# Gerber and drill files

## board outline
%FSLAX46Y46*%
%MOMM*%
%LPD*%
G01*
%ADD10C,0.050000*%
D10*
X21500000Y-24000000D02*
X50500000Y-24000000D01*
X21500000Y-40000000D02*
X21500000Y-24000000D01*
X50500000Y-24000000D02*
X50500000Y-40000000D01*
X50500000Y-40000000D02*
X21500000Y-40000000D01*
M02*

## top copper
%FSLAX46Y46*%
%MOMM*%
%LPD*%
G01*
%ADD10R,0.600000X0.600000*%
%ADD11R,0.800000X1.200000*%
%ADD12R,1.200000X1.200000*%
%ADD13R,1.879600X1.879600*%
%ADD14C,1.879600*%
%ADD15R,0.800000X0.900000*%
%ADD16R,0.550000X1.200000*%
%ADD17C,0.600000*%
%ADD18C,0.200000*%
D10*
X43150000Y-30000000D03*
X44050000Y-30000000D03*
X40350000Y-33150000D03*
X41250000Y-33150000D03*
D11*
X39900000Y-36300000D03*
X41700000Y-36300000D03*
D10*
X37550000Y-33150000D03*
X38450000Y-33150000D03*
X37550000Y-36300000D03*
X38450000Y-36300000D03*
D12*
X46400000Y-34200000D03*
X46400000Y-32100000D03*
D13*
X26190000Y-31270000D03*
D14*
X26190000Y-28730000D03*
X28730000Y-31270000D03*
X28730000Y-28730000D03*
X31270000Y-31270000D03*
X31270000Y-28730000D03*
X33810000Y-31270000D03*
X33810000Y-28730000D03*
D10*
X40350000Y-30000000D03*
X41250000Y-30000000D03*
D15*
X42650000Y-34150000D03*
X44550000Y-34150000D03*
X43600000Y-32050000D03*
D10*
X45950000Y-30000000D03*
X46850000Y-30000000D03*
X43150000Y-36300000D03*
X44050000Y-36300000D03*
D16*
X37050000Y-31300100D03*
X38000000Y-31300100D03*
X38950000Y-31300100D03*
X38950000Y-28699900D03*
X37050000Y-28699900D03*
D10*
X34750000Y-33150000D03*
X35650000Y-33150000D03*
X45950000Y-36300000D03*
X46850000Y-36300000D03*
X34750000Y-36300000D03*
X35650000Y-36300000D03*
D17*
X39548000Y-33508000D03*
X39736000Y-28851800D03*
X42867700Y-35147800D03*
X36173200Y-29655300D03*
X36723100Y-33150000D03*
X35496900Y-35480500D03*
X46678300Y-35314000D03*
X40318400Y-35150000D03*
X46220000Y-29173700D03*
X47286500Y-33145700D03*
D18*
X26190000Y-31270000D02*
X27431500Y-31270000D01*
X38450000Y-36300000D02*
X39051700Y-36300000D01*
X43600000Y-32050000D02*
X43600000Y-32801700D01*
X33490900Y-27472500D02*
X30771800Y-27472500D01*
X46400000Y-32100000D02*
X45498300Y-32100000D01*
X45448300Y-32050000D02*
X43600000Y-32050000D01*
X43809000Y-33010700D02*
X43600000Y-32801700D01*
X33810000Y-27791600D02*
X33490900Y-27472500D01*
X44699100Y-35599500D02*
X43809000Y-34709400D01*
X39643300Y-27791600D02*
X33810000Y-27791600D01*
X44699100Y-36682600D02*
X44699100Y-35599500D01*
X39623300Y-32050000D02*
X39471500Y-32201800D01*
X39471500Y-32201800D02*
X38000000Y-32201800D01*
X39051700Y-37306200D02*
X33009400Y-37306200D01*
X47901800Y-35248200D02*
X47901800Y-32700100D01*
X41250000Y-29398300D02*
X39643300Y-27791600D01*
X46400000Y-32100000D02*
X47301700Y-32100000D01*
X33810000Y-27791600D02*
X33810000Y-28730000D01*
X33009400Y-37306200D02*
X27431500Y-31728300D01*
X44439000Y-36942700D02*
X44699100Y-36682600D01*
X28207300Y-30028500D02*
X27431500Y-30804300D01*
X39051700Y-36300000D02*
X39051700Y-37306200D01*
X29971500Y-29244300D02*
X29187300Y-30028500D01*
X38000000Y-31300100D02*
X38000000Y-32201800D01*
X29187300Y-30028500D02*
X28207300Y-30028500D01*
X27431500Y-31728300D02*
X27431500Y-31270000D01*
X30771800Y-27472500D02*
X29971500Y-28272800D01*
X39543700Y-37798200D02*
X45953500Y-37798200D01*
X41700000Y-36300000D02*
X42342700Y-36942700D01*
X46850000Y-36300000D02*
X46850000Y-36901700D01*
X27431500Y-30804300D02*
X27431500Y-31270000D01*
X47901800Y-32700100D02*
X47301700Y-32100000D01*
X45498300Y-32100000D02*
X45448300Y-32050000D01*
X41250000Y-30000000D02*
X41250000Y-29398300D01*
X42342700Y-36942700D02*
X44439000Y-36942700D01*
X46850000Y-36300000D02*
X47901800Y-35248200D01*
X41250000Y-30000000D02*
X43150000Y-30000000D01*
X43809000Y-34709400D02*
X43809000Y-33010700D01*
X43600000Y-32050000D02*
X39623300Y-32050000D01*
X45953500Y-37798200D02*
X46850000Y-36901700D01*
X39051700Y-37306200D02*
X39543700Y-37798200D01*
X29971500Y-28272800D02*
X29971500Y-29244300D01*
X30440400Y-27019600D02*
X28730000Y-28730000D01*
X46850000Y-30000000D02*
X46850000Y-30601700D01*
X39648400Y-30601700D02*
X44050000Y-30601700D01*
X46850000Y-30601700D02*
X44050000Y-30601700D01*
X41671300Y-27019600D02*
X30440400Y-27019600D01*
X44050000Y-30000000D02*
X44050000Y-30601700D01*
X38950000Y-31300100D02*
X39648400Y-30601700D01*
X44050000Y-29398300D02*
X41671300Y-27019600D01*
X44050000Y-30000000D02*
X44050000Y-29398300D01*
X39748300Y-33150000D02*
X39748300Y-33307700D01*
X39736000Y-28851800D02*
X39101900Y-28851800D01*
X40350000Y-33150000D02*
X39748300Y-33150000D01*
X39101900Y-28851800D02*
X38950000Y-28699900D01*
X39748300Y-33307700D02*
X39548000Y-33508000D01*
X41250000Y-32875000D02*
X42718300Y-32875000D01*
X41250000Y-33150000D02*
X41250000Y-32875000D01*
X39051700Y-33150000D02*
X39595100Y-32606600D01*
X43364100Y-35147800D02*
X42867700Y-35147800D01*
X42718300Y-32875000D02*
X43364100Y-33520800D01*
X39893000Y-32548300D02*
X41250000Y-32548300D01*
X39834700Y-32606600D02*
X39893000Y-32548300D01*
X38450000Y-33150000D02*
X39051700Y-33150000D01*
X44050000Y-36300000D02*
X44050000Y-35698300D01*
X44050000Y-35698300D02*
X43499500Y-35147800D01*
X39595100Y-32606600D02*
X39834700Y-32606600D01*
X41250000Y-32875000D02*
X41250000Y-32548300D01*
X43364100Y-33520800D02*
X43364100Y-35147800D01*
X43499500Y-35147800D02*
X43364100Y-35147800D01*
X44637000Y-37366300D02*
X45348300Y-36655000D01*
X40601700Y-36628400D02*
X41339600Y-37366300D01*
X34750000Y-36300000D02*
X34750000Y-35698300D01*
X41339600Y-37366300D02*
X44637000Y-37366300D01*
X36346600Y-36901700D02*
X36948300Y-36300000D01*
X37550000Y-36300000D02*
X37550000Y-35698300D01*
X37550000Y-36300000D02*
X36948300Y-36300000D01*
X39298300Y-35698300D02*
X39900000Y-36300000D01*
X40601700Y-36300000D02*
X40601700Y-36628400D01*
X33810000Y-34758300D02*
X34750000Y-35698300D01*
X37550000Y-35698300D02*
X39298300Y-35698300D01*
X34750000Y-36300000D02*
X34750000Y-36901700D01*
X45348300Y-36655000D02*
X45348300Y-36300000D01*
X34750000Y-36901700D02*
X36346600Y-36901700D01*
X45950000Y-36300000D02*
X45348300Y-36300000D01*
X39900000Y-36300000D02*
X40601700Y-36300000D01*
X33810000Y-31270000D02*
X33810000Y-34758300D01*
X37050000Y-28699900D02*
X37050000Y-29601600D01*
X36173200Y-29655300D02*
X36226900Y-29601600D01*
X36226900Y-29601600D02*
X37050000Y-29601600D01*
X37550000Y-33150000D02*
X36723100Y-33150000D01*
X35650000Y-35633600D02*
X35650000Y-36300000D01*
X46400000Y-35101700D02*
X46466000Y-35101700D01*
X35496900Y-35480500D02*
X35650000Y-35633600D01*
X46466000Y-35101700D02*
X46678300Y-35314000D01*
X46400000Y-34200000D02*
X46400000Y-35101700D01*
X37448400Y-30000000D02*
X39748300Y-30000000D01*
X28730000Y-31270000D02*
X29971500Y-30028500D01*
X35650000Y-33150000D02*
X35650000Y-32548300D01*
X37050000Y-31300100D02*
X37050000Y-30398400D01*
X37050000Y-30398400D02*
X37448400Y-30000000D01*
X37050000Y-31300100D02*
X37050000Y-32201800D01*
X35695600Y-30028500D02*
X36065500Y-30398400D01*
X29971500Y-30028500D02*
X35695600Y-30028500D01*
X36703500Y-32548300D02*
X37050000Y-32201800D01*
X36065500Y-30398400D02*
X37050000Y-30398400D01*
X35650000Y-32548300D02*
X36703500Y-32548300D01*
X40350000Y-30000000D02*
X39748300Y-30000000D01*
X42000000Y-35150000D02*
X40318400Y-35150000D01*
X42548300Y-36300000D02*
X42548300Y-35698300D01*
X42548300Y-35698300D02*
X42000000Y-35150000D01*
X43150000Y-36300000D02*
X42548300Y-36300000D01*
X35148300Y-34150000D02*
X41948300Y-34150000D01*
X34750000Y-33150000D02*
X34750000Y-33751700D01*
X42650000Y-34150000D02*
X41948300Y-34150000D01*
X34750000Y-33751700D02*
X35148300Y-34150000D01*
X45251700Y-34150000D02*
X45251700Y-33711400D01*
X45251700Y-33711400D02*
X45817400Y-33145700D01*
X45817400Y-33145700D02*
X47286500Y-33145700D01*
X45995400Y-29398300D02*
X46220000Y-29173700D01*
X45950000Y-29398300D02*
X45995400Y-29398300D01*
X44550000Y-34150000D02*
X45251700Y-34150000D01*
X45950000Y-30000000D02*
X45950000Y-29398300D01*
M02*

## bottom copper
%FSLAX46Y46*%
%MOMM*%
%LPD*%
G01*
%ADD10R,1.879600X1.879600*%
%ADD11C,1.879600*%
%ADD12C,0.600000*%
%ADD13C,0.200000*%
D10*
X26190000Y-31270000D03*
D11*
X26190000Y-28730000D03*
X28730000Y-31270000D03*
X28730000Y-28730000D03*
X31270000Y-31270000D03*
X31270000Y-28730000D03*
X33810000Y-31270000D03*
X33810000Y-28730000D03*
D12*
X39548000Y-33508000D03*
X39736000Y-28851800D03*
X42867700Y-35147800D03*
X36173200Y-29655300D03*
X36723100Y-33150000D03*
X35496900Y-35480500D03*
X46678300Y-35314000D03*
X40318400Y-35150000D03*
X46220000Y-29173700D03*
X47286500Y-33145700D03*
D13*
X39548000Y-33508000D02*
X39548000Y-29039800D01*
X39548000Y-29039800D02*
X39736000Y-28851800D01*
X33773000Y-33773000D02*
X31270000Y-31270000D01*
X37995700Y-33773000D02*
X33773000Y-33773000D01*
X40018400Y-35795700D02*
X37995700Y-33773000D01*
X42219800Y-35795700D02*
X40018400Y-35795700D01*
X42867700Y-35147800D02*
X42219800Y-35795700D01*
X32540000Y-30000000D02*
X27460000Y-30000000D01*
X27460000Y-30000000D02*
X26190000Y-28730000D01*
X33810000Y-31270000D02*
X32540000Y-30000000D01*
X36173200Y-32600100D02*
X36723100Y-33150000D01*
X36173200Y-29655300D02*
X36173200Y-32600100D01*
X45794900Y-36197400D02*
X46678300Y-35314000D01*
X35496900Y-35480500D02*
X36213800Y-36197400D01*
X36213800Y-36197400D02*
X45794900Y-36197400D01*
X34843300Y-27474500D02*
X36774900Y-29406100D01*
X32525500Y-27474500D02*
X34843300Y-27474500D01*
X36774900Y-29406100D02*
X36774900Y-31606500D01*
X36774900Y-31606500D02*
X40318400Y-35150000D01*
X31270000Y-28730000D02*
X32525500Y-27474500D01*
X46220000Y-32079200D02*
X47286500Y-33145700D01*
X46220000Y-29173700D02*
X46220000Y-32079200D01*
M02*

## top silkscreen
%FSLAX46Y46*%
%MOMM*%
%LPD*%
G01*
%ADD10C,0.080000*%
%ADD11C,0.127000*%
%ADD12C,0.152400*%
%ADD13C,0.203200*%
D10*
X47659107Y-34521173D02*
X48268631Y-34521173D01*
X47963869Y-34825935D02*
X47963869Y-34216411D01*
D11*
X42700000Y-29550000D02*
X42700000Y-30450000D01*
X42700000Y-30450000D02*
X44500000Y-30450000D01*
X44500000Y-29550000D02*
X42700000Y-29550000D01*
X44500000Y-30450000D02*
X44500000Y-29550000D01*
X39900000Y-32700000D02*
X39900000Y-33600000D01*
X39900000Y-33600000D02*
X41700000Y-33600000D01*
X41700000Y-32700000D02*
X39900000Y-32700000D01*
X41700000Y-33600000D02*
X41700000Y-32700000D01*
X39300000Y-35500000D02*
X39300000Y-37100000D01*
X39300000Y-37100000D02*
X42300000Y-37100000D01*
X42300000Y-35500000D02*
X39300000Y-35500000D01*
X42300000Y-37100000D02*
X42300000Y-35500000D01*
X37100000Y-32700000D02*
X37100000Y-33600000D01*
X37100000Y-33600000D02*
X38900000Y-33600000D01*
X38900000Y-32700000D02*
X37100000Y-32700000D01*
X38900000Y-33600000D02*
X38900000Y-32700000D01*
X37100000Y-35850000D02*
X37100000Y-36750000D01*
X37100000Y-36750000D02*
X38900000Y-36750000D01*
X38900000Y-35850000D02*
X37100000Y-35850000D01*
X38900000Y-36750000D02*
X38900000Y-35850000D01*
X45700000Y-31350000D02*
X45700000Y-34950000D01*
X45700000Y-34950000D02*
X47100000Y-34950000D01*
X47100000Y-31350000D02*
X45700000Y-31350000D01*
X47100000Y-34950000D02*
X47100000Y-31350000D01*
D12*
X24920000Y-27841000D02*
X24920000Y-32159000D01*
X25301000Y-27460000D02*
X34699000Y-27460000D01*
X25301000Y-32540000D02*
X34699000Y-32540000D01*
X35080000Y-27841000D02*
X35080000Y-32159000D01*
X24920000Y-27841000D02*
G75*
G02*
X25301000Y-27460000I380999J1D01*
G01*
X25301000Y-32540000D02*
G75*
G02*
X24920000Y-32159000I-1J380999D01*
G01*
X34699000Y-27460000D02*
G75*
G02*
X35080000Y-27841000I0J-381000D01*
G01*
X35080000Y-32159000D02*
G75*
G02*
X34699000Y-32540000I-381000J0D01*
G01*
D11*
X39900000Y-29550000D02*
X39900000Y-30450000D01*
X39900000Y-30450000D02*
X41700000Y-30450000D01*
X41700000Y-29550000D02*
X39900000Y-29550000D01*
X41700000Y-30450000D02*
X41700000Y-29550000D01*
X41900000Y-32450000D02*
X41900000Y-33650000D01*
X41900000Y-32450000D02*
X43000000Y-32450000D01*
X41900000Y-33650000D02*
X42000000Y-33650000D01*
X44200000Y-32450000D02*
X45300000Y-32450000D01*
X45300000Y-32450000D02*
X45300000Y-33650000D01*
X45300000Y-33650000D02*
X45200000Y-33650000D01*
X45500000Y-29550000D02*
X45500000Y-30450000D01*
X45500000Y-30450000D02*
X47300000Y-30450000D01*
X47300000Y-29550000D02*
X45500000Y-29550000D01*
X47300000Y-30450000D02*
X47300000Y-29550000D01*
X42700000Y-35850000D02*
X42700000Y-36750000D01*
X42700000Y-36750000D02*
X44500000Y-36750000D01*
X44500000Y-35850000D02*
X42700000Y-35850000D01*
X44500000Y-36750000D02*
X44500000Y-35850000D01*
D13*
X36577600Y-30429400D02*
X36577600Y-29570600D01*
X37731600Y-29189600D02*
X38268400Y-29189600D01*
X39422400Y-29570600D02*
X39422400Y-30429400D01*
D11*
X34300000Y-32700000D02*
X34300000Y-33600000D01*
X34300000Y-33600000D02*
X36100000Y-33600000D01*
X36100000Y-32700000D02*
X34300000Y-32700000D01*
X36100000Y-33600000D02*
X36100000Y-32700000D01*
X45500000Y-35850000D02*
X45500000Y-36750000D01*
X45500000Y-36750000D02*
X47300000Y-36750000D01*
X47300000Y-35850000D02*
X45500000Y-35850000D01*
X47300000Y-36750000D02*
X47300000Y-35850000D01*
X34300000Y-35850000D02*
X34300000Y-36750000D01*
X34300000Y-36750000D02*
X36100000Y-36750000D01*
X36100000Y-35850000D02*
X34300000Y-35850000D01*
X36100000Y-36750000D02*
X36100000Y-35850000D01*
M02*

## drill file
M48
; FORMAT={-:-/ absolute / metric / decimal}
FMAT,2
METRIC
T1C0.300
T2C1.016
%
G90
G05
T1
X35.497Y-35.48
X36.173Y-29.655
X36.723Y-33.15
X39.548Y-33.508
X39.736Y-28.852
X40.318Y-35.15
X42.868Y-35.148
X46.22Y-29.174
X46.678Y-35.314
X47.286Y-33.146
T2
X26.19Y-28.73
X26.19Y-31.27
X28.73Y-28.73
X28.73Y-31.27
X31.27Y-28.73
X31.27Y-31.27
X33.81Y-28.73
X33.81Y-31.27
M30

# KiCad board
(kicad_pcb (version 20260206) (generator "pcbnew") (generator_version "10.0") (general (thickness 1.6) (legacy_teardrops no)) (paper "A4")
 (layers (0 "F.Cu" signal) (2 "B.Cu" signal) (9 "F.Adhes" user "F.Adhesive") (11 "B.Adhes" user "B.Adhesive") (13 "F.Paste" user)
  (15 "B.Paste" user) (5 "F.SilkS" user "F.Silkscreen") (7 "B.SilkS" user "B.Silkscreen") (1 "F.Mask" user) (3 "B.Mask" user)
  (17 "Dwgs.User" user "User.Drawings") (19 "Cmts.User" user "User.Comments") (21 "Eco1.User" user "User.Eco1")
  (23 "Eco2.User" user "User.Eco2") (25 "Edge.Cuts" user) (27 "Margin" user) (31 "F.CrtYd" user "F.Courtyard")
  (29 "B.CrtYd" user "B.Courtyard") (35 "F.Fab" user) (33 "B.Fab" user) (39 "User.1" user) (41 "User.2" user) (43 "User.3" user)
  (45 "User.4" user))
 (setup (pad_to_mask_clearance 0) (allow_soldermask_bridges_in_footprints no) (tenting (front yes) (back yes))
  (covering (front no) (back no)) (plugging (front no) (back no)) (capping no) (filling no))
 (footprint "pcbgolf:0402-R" (layer "F.Cu") (at 43.6 30)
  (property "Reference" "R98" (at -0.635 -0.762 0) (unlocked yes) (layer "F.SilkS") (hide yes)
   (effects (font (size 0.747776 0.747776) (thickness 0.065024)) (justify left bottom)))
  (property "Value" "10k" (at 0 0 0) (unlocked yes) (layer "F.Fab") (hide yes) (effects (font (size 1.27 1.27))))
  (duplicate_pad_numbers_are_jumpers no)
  (fp_line (start -0.9 -0.45) (end -0.9 0.45) (stroke (width 0.127) (type solid)) (layer "F.SilkS"))
  (fp_line (start -0.9 0.45) (end 0.9 0.45) (stroke (width 0.127) (type solid)) (layer "F.SilkS"))
  (fp_line (start 0.9 -0.45) (end -0.9 -0.45) (stroke (width 0.127) (type solid)) (layer "F.SilkS"))
  (fp_line (start 0.9 0.45) (end 0.9 -0.45) (stroke (width 0.127) (type solid)) (layer "F.SilkS"))
  (pad "1" smd rect (at -0.45 0) (size 0.6 0.6) (layers "F.Cu" "F.Mask" "F.Paste") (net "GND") (solder_mask_margin 0.0508)
   (solder_paste_margin 0) (thermal_bridge_angle 0))
  (pad "2" smd rect (at 0.45 0) (size 0.6 0.6) (layers "F.Cu" "F.Mask" "F.Paste") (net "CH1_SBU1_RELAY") (solder_mask_margin 0.0508)
   (solder_paste_margin 0) (thermal_bridge_angle 0)))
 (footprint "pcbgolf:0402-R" (layer "F.Cu") (at 40.8 33.15)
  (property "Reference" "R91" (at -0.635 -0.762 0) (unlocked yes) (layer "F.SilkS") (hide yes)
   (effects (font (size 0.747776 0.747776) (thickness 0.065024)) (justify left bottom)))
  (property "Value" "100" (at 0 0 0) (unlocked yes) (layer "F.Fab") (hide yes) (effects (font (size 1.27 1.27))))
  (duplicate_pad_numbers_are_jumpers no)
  (fp_line (start -0.9 -0.45) (end -0.9 0.45) (stroke (width 0.127) (type solid)) (layer "F.SilkS"))
  (fp_line (start -0.9 0.45) (end 0.9 0.45) (stroke (width 0.127) (type solid)) (layer "F.SilkS"))
  (fp_line (start 0.9 -0.45) (end -0.9 -0.45) (stroke (width 0.127) (type solid)) (layer "F.SilkS"))
  (fp_line (start 0.9 0.45) (end 0.9 -0.45) (stroke (width 0.127) (type solid)) (layer "F.SilkS"))
  (pad "1" smd rect (at -0.45 0) (size 0.6 0.6) (layers "F.Cu" "F.Mask" "F.Paste") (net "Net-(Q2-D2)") (solder_mask_margin 0.0508)
   (solder_paste_margin 0) (thermal_bridge_angle 0))
  (pad "2" smd rect (at 0.45 0) (size 0.6 0.6) (layers "F.Cu" "F.Mask" "F.Paste") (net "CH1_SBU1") (solder_mask_margin 0.0508)
   (solder_paste_margin 0) (thermal_bridge_angle 0)))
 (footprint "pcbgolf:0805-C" (layer "F.Cu") (at 40.8 36.3)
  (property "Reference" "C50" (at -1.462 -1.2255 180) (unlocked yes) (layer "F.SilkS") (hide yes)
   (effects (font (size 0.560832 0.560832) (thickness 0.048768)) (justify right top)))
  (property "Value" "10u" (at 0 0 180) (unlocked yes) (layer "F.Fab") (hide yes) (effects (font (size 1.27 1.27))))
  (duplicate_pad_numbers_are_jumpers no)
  (fp_line (start -1.5 -0.8) (end -1.5 0.8) (stroke (width 0.127) (type solid)) (layer "F.SilkS"))
  (fp_line (start -1.5 0.8) (end 1.5 0.8) (stroke (width 0.127) (type solid)) (layer "F.SilkS"))
  (fp_line (start 1.5 -0.8) (end -1.5 -0.8) (stroke (width 0.127) (type solid)) (layer "F.SilkS"))
  (fp_line (start 1.5 0.8) (end 1.5 -0.8) (stroke (width 0.127) (type solid)) (layer "F.SilkS"))
  (pad "1" smd rect (at -0.9 0) (size 0.8 1.2) (layers "F.Cu" "F.Mask" "F.Paste") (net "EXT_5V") (solder_mask_margin 0.0508)
   (solder_paste_margin 0) (thermal_bridge_angle 0))
  (pad "2" smd rect (at 0.9 0) (size 0.8 1.2) (layers "F.Cu" "F.Mask" "F.Paste") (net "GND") (solder_mask_margin 0.0508)
   (solder_paste_margin 0) (thermal_bridge_angle 0)))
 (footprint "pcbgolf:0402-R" (layer "F.Cu") (at 38 33.15)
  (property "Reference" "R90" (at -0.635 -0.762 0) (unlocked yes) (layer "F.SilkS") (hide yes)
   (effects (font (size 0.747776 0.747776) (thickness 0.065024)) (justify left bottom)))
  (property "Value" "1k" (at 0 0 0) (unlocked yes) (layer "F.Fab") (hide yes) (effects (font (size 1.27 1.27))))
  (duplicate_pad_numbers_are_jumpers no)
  (fp_line (start -0.9 -0.45) (end -0.9 0.45) (stroke (width 0.127) (type solid)) (layer "F.SilkS"))
  (fp_line (start -0.9 0.45) (end 0.9 0.45) (stroke (width 0.127) (type solid)) (layer "F.SilkS"))
  (fp_line (start 0.9 -0.45) (end -0.9 -0.45) (stroke (width 0.127) (type solid)) (layer "F.SilkS"))
  (fp_line (start 0.9 0.45) (end 0.9 -0.45) (stroke (width 0.127) (type solid)) (layer "F.SilkS"))
  (pad "1" smd rect (at -0.45 0) (size 0.6 0.6) (layers "F.Cu" "F.Mask" "F.Paste") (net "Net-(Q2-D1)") (solder_mask_margin 0.0508)
   (solder_paste_margin 0) (thermal_bridge_angle 0))
  (pad "2" smd rect (at 0.45 0) (size 0.6 0.6) (layers "F.Cu" "F.Mask" "F.Paste") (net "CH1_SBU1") (solder_mask_margin 0.0508)
   (solder_paste_margin 0) (thermal_bridge_angle 0)))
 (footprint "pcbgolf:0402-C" (layer "F.Cu") (at 38 36.3)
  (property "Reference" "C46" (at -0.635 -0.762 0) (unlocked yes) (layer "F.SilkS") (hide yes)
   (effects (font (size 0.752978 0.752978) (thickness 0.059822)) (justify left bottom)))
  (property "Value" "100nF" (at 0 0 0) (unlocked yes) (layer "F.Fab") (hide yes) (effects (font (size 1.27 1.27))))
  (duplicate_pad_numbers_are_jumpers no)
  (fp_line (start -0.9 -0.45) (end -0.9 0.45) (stroke (width 0.127) (type solid)) (layer "F.SilkS"))
  (fp_line (start -0.9 0.45) (end 0.9 0.45) (stroke (width 0.127) (type solid)) (layer "F.SilkS"))
  (fp_line (start 0.9 -0.45) (end -0.9 -0.45) (stroke (width 0.127) (type solid)) (layer "F.SilkS"))
  (fp_line (start 0.9 0.45) (end 0.9 -0.45) (stroke (width 0.127) (type solid)) (layer "F.SilkS"))
  (pad "1" smd rect (at -0.45 0) (size 0.6 0.6) (layers "F.Cu" "F.Mask" "F.Paste") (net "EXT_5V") (solder_mask_margin 0.0508)
   (solder_paste_margin 0) (thermal_bridge_angle 0))
  (pad "2" smd rect (at 0.45 0) (size 0.6 0.6) (layers "F.Cu" "F.Mask" "F.Paste") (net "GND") (solder_mask_margin 0.0508)
   (solder_paste_margin 0) (thermal_bridge_angle 0)))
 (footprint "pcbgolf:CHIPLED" (layer "F.Cu") (at 46.4 33.15)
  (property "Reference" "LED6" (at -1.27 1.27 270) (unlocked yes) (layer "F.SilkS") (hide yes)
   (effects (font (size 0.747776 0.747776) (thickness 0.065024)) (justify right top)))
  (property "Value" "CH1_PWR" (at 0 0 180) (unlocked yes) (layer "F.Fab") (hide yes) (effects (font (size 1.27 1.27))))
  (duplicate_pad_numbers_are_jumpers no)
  (fp_line (start -0.7 -1.8) (end -0.7 1.8) (stroke (width 0.127) (type solid)) (layer "F.SilkS"))
  (fp_line (start -0.7 1.8) (end 0.7 1.8) (stroke (width 0.127) (type solid)) (layer "F.SilkS"))
  (fp_line (start 0.7 -1.8) (end -0.7 -1.8) (stroke (width 0.127) (type solid)) (layer "F.SilkS"))
  (fp_line (start 0.7 1.8) (end 0.7 -1.8) (stroke (width 0.127) (type solid)) (layer "F.SilkS"))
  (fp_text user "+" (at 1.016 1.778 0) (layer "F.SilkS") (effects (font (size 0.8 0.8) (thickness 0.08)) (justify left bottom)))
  (pad "A" smd rect (at 0 1.05) (size 1.2 1.2) (layers "F.Cu" "F.Mask" "F.Paste") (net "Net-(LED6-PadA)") (solder_mask_margin 0.0508)
   (solder_paste_margin 0) (thermal_bridge_angle 0))
  (pad "C" smd rect (at 0 -1.05) (size 1.2 1.2) (layers "F.Cu" "F.Mask" "F.Paste") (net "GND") (solder_mask_margin 0.0508)
   (solder_paste_margin 0) (thermal_bridge_angle 0)))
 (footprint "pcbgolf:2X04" (layer "F.Cu") (at 30 30)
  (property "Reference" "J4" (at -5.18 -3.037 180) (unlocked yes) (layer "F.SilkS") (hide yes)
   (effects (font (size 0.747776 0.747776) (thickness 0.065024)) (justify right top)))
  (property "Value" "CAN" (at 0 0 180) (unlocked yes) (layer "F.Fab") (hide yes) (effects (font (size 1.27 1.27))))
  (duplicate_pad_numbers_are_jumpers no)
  (fp_line (start -5.08 -2.159) (end -5.08 2.159) (stroke (width 0.1524) (type solid)) (layer "F.SilkS"))
  (fp_line (start -4.699 -2.54) (end 4.699 -2.54) (stroke (width 0.1524) (type solid)) (layer "F.SilkS"))
  (fp_line (start -4.699 2.54) (end 4.699 2.54) (stroke (width 0.1524) (type solid)) (layer "F.SilkS"))
  (fp_line (start 5.08 -2.159) (end 5.08 2.159) (stroke (width 0.1524) (type solid)) (layer "F.SilkS"))
  (fp_arc (start -5.08 -2.159) (mid -4.968408 -2.428408) (end -4.699 -2.54) (stroke (width 0.1524) (type solid)) (layer "F.SilkS"))
  (fp_arc (start -4.699 2.54) (mid -4.968408 2.428408) (end -5.08 2.159) (stroke (width 0.1524) (type solid)) (layer "F.SilkS"))
  (fp_arc (start 4.699 -2.54) (mid 4.968408 -2.428408) (end 5.08 -2.159) (stroke (width 0.1524) (type solid)) (layer "F.SilkS"))
  (fp_arc (start 5.08 2.159) (mid 4.968408 2.428408) (end 4.699 2.54) (stroke (width 0.1524) (type solid)) (layer "F.SilkS"))
  (pad "1" thru_hole rect (at -3.81 1.27 90) (size 1.8796 1.8796) (drill 1.016) (layers "*.Cu" "*.Mask") (remove_unused_layers no)
   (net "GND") (solder_mask_margin 0.0508) (thermal_bridge_angle 0))
  (pad "2" thru_hole circle (at -3.81 -1.27 90) (size 1.8796 1.8796) (drill 1.016) (layers "*.Cu" "*.Mask") (remove_unused_layers no)
   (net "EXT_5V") (solder_mask_margin 0.0508) (thermal_bridge_angle 0))
  (pad "3" thru_hole circle (at -1.27 1.27 90) (size 1.8796 1.8796) (drill 1.016) (layers "*.Cu" "*.Mask") (remove_unused_layers no)
   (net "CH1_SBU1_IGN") (solder_mask_margin 0.0508) (thermal_bridge_angle 0))
  (pad "4" thru_hole circle (at -1.27 -1.27 90) (size 1.8796 1.8796) (drill 1.016) (layers "*.Cu" "*.Mask") (remove_unused_layers no)
   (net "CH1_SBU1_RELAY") (solder_mask_margin 0.0508) (thermal_bridge_angle 0))
  (pad "5" thru_hole circle (at 1.27 1.27 90) (size 1.8796 1.8796) (drill 1.016) (layers "*.Cu" "*.Mask") (remove_unused_layers no)
   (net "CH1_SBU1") (solder_mask_margin 0.0508) (thermal_bridge_angle 0))
  (pad "6" thru_hole circle (at 1.27 -1.27 90) (size 1.8796 1.8796) (drill 1.016) (layers "*.Cu" "*.Mask") (remove_unused_layers no)
   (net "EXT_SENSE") (solder_mask_margin 0.0508) (thermal_bridge_angle 0))
  (pad "7" thru_hole circle (at 3.81 1.27 90) (size 1.8796 1.8796) (drill 1.016) (layers "*.Cu" "*.Mask") (remove_unused_layers no)
   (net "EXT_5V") (solder_mask_margin 0.0508) (thermal_bridge_angle 0))
  (pad "8" thru_hole circle (at 3.81 -1.27 90) (size 1.8796 1.8796) (drill 1.016) (layers "*.Cu" "*.Mask") (remove_unused_layers no)
   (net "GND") (solder_mask_margin 0.0508) (thermal_bridge_angle 0)))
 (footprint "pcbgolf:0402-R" (layer "F.Cu") (at 40.8 30)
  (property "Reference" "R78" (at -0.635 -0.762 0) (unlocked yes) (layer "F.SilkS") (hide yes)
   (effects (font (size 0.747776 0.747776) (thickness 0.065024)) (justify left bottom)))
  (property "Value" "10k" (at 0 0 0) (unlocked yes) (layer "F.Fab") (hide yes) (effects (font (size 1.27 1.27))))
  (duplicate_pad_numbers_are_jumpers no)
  (fp_line (start -0.9 -0.45) (end -0.9 0.45) (stroke (width 0.127) (type solid)) (layer "F.SilkS"))
  (fp_line (start -0.9 0.45) (end 0.9 0.45) (stroke (width 0.127) (type solid)) (layer "F.SilkS"))
  (fp_line (start 0.9 -0.45) (end -0.9 -0.45) (stroke (width 0.127) (type solid)) (layer "F.SilkS"))
  (fp_line (start 0.9 0.45) (end 0.9 -0.45) (stroke (width 0.127) (type solid)) (layer "F.SilkS"))
  (pad "1" smd rect (at -0.45 0) (size 0.6 0.6) (layers "F.Cu" "F.Mask" "F.Paste") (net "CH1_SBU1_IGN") (solder_mask_margin 0.0508)
   (solder_paste_margin 0) (thermal_bridge_angle 0))
  (pad "2" smd rect (at 0.45 0) (size 0.6 0.6) (layers "F.Cu" "F.Mask" "F.Paste") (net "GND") (solder_mask_margin 0.0508)
   (solder_paste_margin 0) (thermal_bridge_angle 0)))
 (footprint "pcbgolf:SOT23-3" (layer "F.Cu") (at 43.6 33.15)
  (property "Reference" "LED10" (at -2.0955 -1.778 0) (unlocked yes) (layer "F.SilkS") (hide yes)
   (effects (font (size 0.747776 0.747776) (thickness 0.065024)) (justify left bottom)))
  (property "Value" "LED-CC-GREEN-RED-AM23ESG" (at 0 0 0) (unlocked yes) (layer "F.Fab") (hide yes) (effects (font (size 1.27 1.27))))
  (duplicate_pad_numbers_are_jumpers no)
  (fp_line (start -1.7 -0.7) (end -1.7 0.5) (stroke (width 0.127) (type solid)) (layer "F.SilkS"))
  (fp_line (start -1.7 -0.7) (end -0.6 -0.7) (stroke (width 0.127) (type solid)) (layer "F.SilkS"))
  (fp_line (start -1.7 0.5) (end -1.6 0.5) (stroke (width 0.127) (type solid)) (layer "F.SilkS"))
  (fp_line (start 0.6 -0.7) (end 1.7 -0.7) (stroke (width 0.127) (type solid)) (layer "F.SilkS"))
  (fp_line (start 1.7 -0.7) (end 1.7 0.5) (stroke (width 0.127) (type solid)) (layer "F.SilkS"))
  (fp_line (start 1.7 0.5) (end 1.6 0.5) (stroke (width 0.127) (type solid)) (layer "F.SilkS"))
  (pad "1" smd rect (at -0.95 1) (size 0.8 0.9) (layers "F.Cu" "F.Mask" "F.Paste") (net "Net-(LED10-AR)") (solder_mask_margin 0.0508)
   (solder_paste_margin 0) (thermal_bridge_angle 0))
  (pad "2" smd rect (at 0.95 1) (size 0.8 0.9) (layers "F.Cu" "F.Mask" "F.Paste") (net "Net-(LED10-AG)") (solder_mask_margin 0.0508)
   (solder_paste_margin 0) (thermal_bridge_angle 0))
  (pad "3" smd rect (at 0 -1.1) (size 0.8 0.9) (layers "F.Cu" "F.Mask" "F.Paste") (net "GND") (solder_mask_margin 0.0508)
   (solder_paste_margin 0) (thermal_bridge_angle 0)))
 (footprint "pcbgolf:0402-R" (layer "F.Cu") (at 46.4 30)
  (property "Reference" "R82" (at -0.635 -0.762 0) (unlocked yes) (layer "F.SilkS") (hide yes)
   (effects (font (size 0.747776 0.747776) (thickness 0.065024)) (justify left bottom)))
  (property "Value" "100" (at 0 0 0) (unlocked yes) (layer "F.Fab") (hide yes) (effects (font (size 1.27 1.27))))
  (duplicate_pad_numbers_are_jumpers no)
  (fp_line (start -0.9 -0.45) (end -0.9 0.45) (stroke (width 0.127) (type solid)) (layer "F.SilkS"))
  (fp_line (start -0.9 0.45) (end 0.9 0.45) (stroke (width 0.127) (type solid)) (layer "F.SilkS"))
  (fp_line (start 0.9 -0.45) (end -0.9 -0.45) (stroke (width 0.127) (type solid)) (layer "F.SilkS"))
  (fp_line (start 0.9 0.45) (end 0.9 -0.45) (stroke (width 0.127) (type solid)) (layer "F.SilkS"))
  (pad "1" smd rect (at -0.45 0) (size 0.6 0.6) (layers "F.Cu" "F.Mask" "F.Paste") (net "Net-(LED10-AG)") (solder_mask_margin 0.0508)
   (solder_paste_margin 0) (thermal_bridge_angle 0))
  (pad "2" smd rect (at 0.45 0) (size 0.6 0.6) (layers "F.Cu" "F.Mask" "F.Paste") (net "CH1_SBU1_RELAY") (solder_mask_margin 0.0508)
   (solder_paste_margin 0) (thermal_bridge_angle 0)))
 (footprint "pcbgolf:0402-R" (layer "F.Cu") (at 43.6 36.3)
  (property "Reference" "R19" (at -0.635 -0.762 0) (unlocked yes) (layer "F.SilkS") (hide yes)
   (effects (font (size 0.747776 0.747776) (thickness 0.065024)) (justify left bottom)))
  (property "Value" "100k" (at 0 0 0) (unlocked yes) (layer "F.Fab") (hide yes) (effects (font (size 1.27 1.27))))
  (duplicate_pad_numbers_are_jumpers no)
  (fp_line (start -0.9 -0.45) (end -0.9 0.45) (stroke (width 0.127) (type solid)) (layer "F.SilkS"))
  (fp_line (start -0.9 0.45) (end 0.9 0.45) (stroke (width 0.127) (type solid)) (layer "F.SilkS"))
  (fp_line (start 0.9 -0.45) (end -0.9 -0.45) (stroke (width 0.127) (type solid)) (layer "F.SilkS"))
  (fp_line (start 0.9 0.45) (end 0.9 -0.45) (stroke (width 0.127) (type solid)) (layer "F.SilkS"))
  (pad "1" smd rect (at -0.45 0) (size 0.6 0.6) (layers "F.Cu" "F.Mask" "F.Paste") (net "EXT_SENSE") (solder_mask_margin 0.0508)
   (solder_paste_margin 0) (thermal_bridge_angle 0))
  (pad "2" smd rect (at 0.45 0) (size 0.6 0.6) (layers "F.Cu" "F.Mask" "F.Paste") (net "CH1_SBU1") (solder_mask_margin 0.0508)
   (solder_paste_margin 0) (thermal_bridge_angle 0)))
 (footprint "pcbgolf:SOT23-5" (layer "F.Cu") (at 38 30)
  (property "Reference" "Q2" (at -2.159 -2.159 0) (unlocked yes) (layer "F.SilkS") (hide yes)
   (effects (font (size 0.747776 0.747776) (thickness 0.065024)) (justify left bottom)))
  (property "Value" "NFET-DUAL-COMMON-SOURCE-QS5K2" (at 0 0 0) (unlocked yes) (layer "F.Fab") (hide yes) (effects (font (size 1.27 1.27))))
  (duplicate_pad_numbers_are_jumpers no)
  (fp_line (start -1.4224 0.4294) (end -1.4224 -0.4294) (stroke (width 0.2032) (type solid)) (layer "F.SilkS"))
  (fp_line (start -0.2684 -0.8104) (end 0.2684 -0.8104) (stroke (width 0.2032) (type solid)) (layer "F.SilkS"))
  (fp_line (start 1.4224 -0.4294) (end 1.4224 0.4294) (stroke (width 0.2032) (type solid)) (layer "F.SilkS"))
  (pad "1" smd rect (at -0.95 1.3001) (size 0.55 1.2) (layers "F.Cu" "F.Mask" "F.Paste") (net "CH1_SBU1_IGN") (solder_mask_margin 0.0508)
   (solder_paste_margin 0) (thermal_bridge_angle 0))
  (pad "2" smd rect (at 0 1.3001) (size 0.55 1.2) (layers "F.Cu" "F.Mask" "F.Paste") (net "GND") (solder_mask_margin 0.0508)
   (solder_paste_margin 0) (thermal_bridge_angle 0))
  (pad "3" smd rect (at 0.95 1.3001) (size 0.55 1.2) (layers "F.Cu" "F.Mask" "F.Paste") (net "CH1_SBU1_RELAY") (solder_mask_margin 0.0508)
   (solder_paste_margin 0) (thermal_bridge_angle 0))
  (pad "4" smd rect (at 0.95 -1.3001) (size 0.55 1.2) (layers "F.Cu" "F.Mask" "F.Paste") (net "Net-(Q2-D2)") (solder_mask_margin 0.0508)
   (solder_paste_margin 0) (thermal_bridge_angle 0))
  (pad "5" smd rect (at -0.95 -1.3001) (size 0.55 1.2) (layers "F.Cu" "F.Mask" "F.Paste") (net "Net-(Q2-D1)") (solder_mask_margin 0.0508)
   (solder_paste_margin 0) (thermal_bridge_angle 0)))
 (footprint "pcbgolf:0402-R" (layer "F.Cu") (at 35.2 33.15)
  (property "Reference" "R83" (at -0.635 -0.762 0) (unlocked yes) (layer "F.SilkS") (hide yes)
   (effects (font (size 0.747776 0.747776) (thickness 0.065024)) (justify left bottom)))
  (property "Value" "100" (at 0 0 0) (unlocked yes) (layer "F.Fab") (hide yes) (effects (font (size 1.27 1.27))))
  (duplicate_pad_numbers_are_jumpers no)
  (fp_line (start -0.9 -0.45) (end -0.9 0.45) (stroke (width 0.127) (type solid)) (layer "F.SilkS"))
  (fp_line (start -0.9 0.45) (end 0.9 0.45) (stroke (width 0.127) (type solid)) (layer "F.SilkS"))
  (fp_line (start 0.9 -0.45) (end -0.9 -0.45) (stroke (width 0.127) (type solid)) (layer "F.SilkS"))
  (fp_line (start 0.9 0.45) (end 0.9 -0.45) (stroke (width 0.127) (type solid)) (layer "F.SilkS"))
  (pad "1" smd rect (at -0.45 0) (size 0.6 0.6) (layers "F.Cu" "F.Mask" "F.Paste") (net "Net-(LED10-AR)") (solder_mask_margin 0.0508)
   (solder_paste_margin 0) (thermal_bridge_angle 0))
  (pad "2" smd rect (at 0.45 0) (size 0.6 0.6) (layers "F.Cu" "F.Mask" "F.Paste") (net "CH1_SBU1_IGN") (solder_mask_margin 0.0508)
   (solder_paste_margin 0) (thermal_bridge_angle 0)))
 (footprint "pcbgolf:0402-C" (layer "F.Cu") (at 46.4 36.3)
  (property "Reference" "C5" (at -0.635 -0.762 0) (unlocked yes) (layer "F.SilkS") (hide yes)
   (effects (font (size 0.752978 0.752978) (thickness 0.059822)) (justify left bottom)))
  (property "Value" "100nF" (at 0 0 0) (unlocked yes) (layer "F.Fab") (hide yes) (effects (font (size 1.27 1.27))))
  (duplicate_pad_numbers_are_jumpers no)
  (fp_line (start -0.9 -0.45) (end -0.9 0.45) (stroke (width 0.127) (type solid)) (layer "F.SilkS"))
  (fp_line (start -0.9 0.45) (end 0.9 0.45) (stroke (width 0.127) (type solid)) (layer "F.SilkS"))
  (fp_line (start 0.9 -0.45) (end -0.9 -0.45) (stroke (width 0.127) (type solid)) (layer "F.SilkS"))
  (fp_line (start 0.9 0.45) (end 0.9 -0.45) (stroke (width 0.127) (type solid)) (layer "F.SilkS"))
  (pad "1" smd rect (at -0.45 0) (size 0.6 0.6) (layers "F.Cu" "F.Mask" "F.Paste") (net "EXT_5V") (solder_mask_margin 0.0508)
   (solder_paste_margin 0) (thermal_bridge_angle 0))
  (pad "2" smd rect (at 0.45 0) (size 0.6 0.6) (layers "F.Cu" "F.Mask" "F.Paste") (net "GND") (solder_mask_margin 0.0508)
   (solder_paste_margin 0) (thermal_bridge_angle 0)))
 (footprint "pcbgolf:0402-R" (layer "F.Cu") (at 35.2 36.3)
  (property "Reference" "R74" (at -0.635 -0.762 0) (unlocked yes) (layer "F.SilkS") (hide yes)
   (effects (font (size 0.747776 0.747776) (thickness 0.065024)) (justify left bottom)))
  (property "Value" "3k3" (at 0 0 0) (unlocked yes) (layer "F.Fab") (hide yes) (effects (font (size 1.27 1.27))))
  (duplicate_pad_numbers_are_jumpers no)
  (fp_line (start -0.9 -0.45) (end -0.9 0.45) (stroke (width 0.127) (type solid)) (layer "F.SilkS"))
  (fp_line (start -0.9 0.45) (end 0.9 0.45) (stroke (width 0.127) (type solid)) (layer "F.SilkS"))
  (fp_line (start 0.9 -0.45) (end -0.9 -0.45) (stroke (width 0.127) (type solid)) (layer "F.SilkS"))
  (fp_line (start 0.9 0.45) (end 0.9 -0.45) (stroke (width 0.127) (type solid)) (layer "F.SilkS"))
  (pad "1" smd rect (at -0.45 0) (size 0.6 0.6) (layers "F.Cu" "F.Mask" "F.Paste") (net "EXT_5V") (solder_mask_margin 0.0508)
   (solder_paste_margin 0) (thermal_bridge_angle 0))
  (pad "2" smd rect (at 0.45 0) (size 0.6 0.6) (layers "F.Cu" "F.Mask" "F.Paste") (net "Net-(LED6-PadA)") (solder_mask_margin 0.0508)
   (solder_paste_margin 0) (thermal_bridge_angle 0)))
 (gr_line (start 21.5 24) (end 50.5 24) (stroke (width 0.05) (type default)) (layer "Edge.Cuts"))
 (gr_line (start 21.5 40) (end 21.5 24) (stroke (width 0.05) (type default)) (layer "Edge.Cuts"))
 (gr_line (start 50.5 24) (end 50.5 40) (stroke (width 0.05) (type default)) (layer "Edge.Cuts"))
 (gr_line (start 50.5 40) (end 21.5 40) (stroke (width 0.05) (type default)) (layer "Edge.Cuts"))
 (segment (start 26.19 31.27) (end 27.4315 31.27) (width 0.2) (layer "F.Cu") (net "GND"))
 (segment (start 38.45 36.3) (end 39.0517 36.3) (width 0.2) (layer "F.Cu") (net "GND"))
 (segment (start 43.6 32.05) (end 43.6 32.8017) (width 0.2) (layer "F.Cu") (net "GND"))
 (segment (start 33.4909 27.4725) (end 30.7718 27.4725) (width 0.2) (layer "F.Cu") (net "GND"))
 (segment (start 46.4 32.1) (end 45.4983 32.1) (width 0.2) (layer "F.Cu") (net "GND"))
 (segment (start 45.4483 32.05) (end 43.6 32.05) (width 0.2) (layer "F.Cu") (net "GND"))
 (segment (start 43.809 33.0107) (end 43.6 32.8017) (width 0.2) (layer "F.Cu") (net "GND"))
 (segment (start 33.81 27.7916) (end 33.4909 27.4725) (width 0.2) (layer "F.Cu") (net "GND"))
 (segment (start 44.6991 35.5995) (end 43.809 34.7094) (width 0.2) (layer "F.Cu") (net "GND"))
 (segment (start 39.6433 27.7916) (end 33.81 27.7916) (width 0.2) (layer "F.Cu") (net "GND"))
 (segment (start 44.6991 36.6826) (end 44.6991 35.5995) (width 0.2) (layer "F.Cu") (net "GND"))
 (segment (start 39.6233 32.05) (end 39.4715 32.2018) (width 0.2) (layer "F.Cu") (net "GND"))
 (segment (start 39.4715 32.2018) (end 38 32.2018) (width 0.2) (layer "F.Cu") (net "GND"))
 (segment (start 39.0517 37.3062) (end 33.0094 37.3062) (width 0.2) (layer "F.Cu") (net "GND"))
 (segment (start 47.9018 35.2482) (end 47.9018 32.7001) (width 0.2) (layer "F.Cu") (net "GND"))
 (segment (start 41.25 29.3983) (end 39.6433 27.7916) (width 0.2) (layer "F.Cu") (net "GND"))
 (segment (start 46.4 32.1) (end 47.3017 32.1) (width 0.2) (layer "F.Cu") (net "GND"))
 (segment (start 33.81 27.7916) (end 33.81 28.73) (width 0.2) (layer "F.Cu") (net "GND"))
 (segment (start 33.0094 37.3062) (end 27.4315 31.7283) (width 0.2) (layer "F.Cu") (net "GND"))
 (segment (start 44.439 36.9427) (end 44.6991 36.6826) (width 0.2) (layer "F.Cu") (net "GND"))
 (segment (start 28.2073 30.0285) (end 27.4315 30.8043) (width 0.2) (layer "F.Cu") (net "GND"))
 (segment (start 39.0517 36.3) (end 39.0517 37.3062) (width 0.2) (layer "F.Cu") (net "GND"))
 (segment (start 29.9715 29.2443) (end 29.1873 30.0285) (width 0.2) (layer "F.Cu") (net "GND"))
 (segment (start 38 31.3001) (end 38 32.2018) (width 0.2) (layer "F.Cu") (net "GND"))
 (segment (start 29.1873 30.0285) (end 28.2073 30.0285) (width 0.2) (layer "F.Cu") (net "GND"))
 (segment (start 27.4315 31.7283) (end 27.4315 31.27) (width 0.2) (layer "F.Cu") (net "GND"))
 (segment (start 30.7718 27.4725) (end 29.9715 28.2728) (width 0.2) (layer "F.Cu") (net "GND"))
 (segment (start 39.5437 37.7982) (end 45.9535 37.7982) (width 0.2) (layer "F.Cu") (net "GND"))
 (segment (start 41.7 36.3) (end 42.3427 36.9427) (width 0.2) (layer "F.Cu") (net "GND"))
 (segment (start 46.85 36.3) (end 46.85 36.9017) (width 0.2) (layer "F.Cu") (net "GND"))
 (segment (start 27.4315 30.8043) (end 27.4315 31.27) (width 0.2) (layer "F.Cu") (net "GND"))
 (segment (start 47.9018 32.7001) (end 47.3017 32.1) (width 0.2) (layer "F.Cu") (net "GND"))
 (segment (start 45.4983 32.1) (end 45.4483 32.05) (width 0.2) (layer "F.Cu") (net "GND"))
 (segment (start 41.25 30) (end 41.25 29.3983) (width 0.2) (layer "F.Cu") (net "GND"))
 (segment (start 42.3427 36.9427) (end 44.439 36.9427) (width 0.2) (layer "F.Cu") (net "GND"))
 (segment (start 46.85 36.3) (end 47.9018 35.2482) (width 0.2) (layer "F.Cu") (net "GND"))
 (segment (start 41.25 30) (end 43.15 30) (width 0.2) (layer "F.Cu") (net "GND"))
 (segment (start 43.809 34.7094) (end 43.809 33.0107) (width 0.2) (layer "F.Cu") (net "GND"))
 (segment (start 43.6 32.05) (end 39.6233 32.05) (width 0.2) (layer "F.Cu") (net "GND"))
 (segment (start 45.9535 37.7982) (end 46.85 36.9017) (width 0.2) (layer "F.Cu") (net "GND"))
 (segment (start 39.0517 37.3062) (end 39.5437 37.7982) (width 0.2) (layer "F.Cu") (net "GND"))
 (segment (start 29.9715 28.2728) (end 29.9715 29.2443) (width 0.2) (layer "F.Cu") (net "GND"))
 (segment (start 30.4404 27.0196) (end 28.73 28.73) (width 0.2) (layer "F.Cu") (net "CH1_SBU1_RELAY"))
 (segment (start 46.85 30) (end 46.85 30.6017) (width 0.2) (layer "F.Cu") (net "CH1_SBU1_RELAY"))
 (segment (start 39.6484 30.6017) (end 44.05 30.6017) (width 0.2) (layer "F.Cu") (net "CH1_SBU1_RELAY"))
 (segment (start 46.85 30.6017) (end 44.05 30.6017) (width 0.2) (layer "F.Cu") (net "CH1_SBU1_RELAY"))
 (segment (start 41.6713 27.0196) (end 30.4404 27.0196) (width 0.2) (layer "F.Cu") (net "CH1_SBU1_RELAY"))
 (segment (start 44.05 30) (end 44.05 30.6017) (width 0.2) (layer "F.Cu") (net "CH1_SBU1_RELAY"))
 (segment (start 38.95 31.3001) (end 39.6484 30.6017) (width 0.2) (layer "F.Cu") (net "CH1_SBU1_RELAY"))
 (segment (start 44.05 29.3983) (end 41.6713 27.0196) (width 0.2) (layer "F.Cu") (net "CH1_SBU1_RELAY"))
 (segment (start 44.05 30) (end 44.05 29.3983) (width 0.2) (layer "F.Cu") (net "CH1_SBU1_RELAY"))
 (segment (start 39.7483 33.15) (end 39.7483 33.3077) (width 0.2) (layer "F.Cu") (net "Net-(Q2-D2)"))
 (segment (start 39.736 28.8518) (end 39.1019 28.8518) (width 0.2) (layer "F.Cu") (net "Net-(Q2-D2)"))
 (segment (start 40.35 33.15) (end 39.7483 33.15) (width 0.2) (layer "F.Cu") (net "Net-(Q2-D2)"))
 (segment (start 39.1019 28.8518) (end 38.95 28.6999) (width 0.2) (layer "F.Cu") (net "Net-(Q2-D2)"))
 (segment (start 39.7483 33.3077) (end 39.548 33.508) (width 0.2) (layer "F.Cu") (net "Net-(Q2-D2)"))
 (via (at 39.548 33.508) (size 0.6) (drill 0.3) (layers "F.Cu" "B.Cu") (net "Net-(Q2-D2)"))
 (via (at 39.736 28.8518) (size 0.6) (drill 0.3) (layers "F.Cu" "B.Cu") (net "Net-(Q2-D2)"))
 (segment (start 39.548 33.508) (end 39.548 29.0398) (width 0.2) (layer "B.Cu") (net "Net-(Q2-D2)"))
 (segment (start 39.548 29.0398) (end 39.736 28.8518) (width 0.2) (layer "B.Cu") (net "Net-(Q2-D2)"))
 (segment (start 41.25 32.875) (end 42.7183 32.875) (width 0.2) (layer "F.Cu") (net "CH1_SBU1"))
 (segment (start 41.25 33.15) (end 41.25 32.875) (width 0.2) (layer "F.Cu") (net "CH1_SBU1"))
 (segment (start 39.0517 33.15) (end 39.5951 32.6066) (width 0.2) (layer "F.Cu") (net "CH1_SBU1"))
 (segment (start 43.3641 35.1478) (end 42.8677 35.1478) (width 0.2) (layer "F.Cu") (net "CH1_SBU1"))
 (segment (start 42.7183 32.875) (end 43.3641 33.5208) (width 0.2) (layer "F.Cu") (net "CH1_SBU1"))
 (segment (start 39.893 32.5483) (end 41.25 32.5483) (width 0.2) (layer "F.Cu") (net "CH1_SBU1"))
 (segment (start 39.8347 32.6066) (end 39.893 32.5483) (width 0.2) (layer "F.Cu") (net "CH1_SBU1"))
 (segment (start 38.45 33.15) (end 39.0517 33.15) (width 0.2) (layer "F.Cu") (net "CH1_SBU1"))
 (segment (start 44.05 36.3) (end 44.05 35.6983) (width 0.2) (layer "F.Cu") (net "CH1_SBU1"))
 (segment (start 44.05 35.6983) (end 43.4995 35.1478) (width 0.2) (layer "F.Cu") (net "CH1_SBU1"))
 (segment (start 39.5951 32.6066) (end 39.8347 32.6066) (width 0.2) (layer "F.Cu") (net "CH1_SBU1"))
 (segment (start 41.25 32.875) (end 41.25 32.5483) (width 0.2) (layer "F.Cu") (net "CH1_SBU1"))
 (segment (start 43.3641 33.5208) (end 43.3641 35.1478) (width 0.2) (layer "F.Cu") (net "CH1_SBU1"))
 (segment (start 43.4995 35.1478) (end 43.3641 35.1478) (width 0.2) (layer "F.Cu") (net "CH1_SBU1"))
 (via (at 42.8677 35.1478) (size 0.6) (drill 0.3) (layers "F.Cu" "B.Cu") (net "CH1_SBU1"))
 (segment (start 33.773 33.773) (end 31.27 31.27) (width 0.2) (layer "B.Cu") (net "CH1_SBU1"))
 (segment (start 37.9957 33.773) (end 33.773 33.773) (width 0.2) (layer "B.Cu") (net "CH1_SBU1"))
 (segment (start 40.0184 35.7957) (end 37.9957 33.773) (width 0.2) (layer "B.Cu") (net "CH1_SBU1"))
 (segment (start 42.2198 35.7957) (end 40.0184 35.7957) (width 0.2) (layer "B.Cu") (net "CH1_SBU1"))
 (segment (start 42.8677 35.1478) (end 42.2198 35.7957) (width 0.2) (layer "B.Cu") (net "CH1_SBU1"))
 (segment (start 44.637 37.3663) (end 45.3483 36.655) (width 0.2) (layer "F.Cu") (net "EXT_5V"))
 (segment (start 40.6017 36.6284) (end 41.3396 37.3663) (width 0.2) (layer "F.Cu") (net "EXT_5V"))
 (segment (start 34.75 36.3) (end 34.75 35.6983) (width 0.2) (layer "F.Cu") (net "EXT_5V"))
 (segment (start 41.3396 37.3663) (end 44.637 37.3663) (width 0.2) (layer "F.Cu") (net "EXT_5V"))
 (segment (start 36.3466 36.9017) (end 36.9483 36.3) (width 0.2) (layer "F.Cu") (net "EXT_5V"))
 (segment (start 37.55 36.3) (end 37.55 35.6983) (width 0.2) (layer "F.Cu") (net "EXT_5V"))
 (segment (start 37.55 36.3) (end 36.9483 36.3) (width 0.2) (layer "F.Cu") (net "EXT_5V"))
 (segment (start 39.2983 35.6983) (end 39.9 36.3) (width 0.2) (layer "F.Cu") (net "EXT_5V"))
 (segment (start 40.6017 36.3) (end 40.6017 36.6284) (width 0.2) (layer "F.Cu") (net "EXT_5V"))
 (segment (start 33.81 34.7583) (end 34.75 35.6983) (width 0.2) (layer "F.Cu") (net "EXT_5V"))
 (segment (start 37.55 35.6983) (end 39.2983 35.6983) (width 0.2) (layer "F.Cu") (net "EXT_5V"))
 (segment (start 34.75 36.3) (end 34.75 36.9017) (width 0.2) (layer "F.Cu") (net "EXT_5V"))
 (segment (start 45.3483 36.655) (end 45.3483 36.3) (width 0.2) (layer "F.Cu") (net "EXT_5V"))
 (segment (start 34.75 36.9017) (end 36.3466 36.9017) (width 0.2) (layer "F.Cu") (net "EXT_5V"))
 (segment (start 45.95 36.3) (end 45.3483 36.3) (width 0.2) (layer "F.Cu") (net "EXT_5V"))
 (segment (start 39.9 36.3) (end 40.6017 36.3) (width 0.2) (layer "F.Cu") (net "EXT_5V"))
 (segment (start 33.81 31.27) (end 33.81 34.7583) (width 0.2) (layer "F.Cu") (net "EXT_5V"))
 (segment (start 32.54 30) (end 27.46 30) (width 0.2) (layer "B.Cu") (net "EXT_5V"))
 (segment (start 27.46 30) (end 26.19 28.73) (width 0.2) (layer "B.Cu") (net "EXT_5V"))
 (segment (start 33.81 31.27) (end 32.54 30) (width 0.2) (layer "B.Cu") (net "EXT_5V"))
 (segment (start 37.05 28.6999) (end 37.05 29.6016) (width 0.2) (layer "F.Cu") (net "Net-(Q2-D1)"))
 (segment (start 36.1732 29.6553) (end 36.2269 29.6016) (width 0.2) (layer "F.Cu") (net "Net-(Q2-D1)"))
 (segment (start 36.2269 29.6016) (end 37.05 29.6016) (width 0.2) (layer "F.Cu") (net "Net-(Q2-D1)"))
 (segment (start 37.55 33.15) (end 36.7231 33.15) (width 0.2) (layer "F.Cu") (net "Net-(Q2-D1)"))
 (via (at 36.1732 29.6553) (size 0.6) (drill 0.3) (layers "F.Cu" "B.Cu") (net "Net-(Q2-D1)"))
 (via (at 36.7231 33.15) (size 0.6) (drill 0.3) (layers "F.Cu" "B.Cu") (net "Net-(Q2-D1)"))
 (segment (start 36.1732 32.6001) (end 36.7231 33.15) (width 0.2) (layer "B.Cu") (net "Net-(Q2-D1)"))
 (segment (start 36.1732 29.6553) (end 36.1732 32.6001) (width 0.2) (layer "B.Cu") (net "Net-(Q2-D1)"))
 (segment (start 35.65 35.6336) (end 35.65 36.3) (width 0.2) (layer "F.Cu") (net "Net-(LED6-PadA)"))
 (segment (start 46.4 35.1017) (end 46.466 35.1017) (width 0.2) (layer "F.Cu") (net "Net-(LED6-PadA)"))
 (segment (start 35.4969 35.4805) (end 35.65 35.6336) (width 0.2) (layer "F.Cu") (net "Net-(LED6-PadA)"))
 (segment (start 46.466 35.1017) (end 46.6783 35.314) (width 0.2) (layer "F.Cu") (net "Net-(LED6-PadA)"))
 (segment (start 46.4 34.2) (end 46.4 35.1017) (width 0.2) (layer "F.Cu") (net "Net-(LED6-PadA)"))
 (via (at 35.4969 35.4805) (size 0.6) (drill 0.3) (layers "F.Cu" "B.Cu") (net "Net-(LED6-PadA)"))
 (via (at 46.6783 35.314) (size 0.6) (drill 0.3) (layers "F.Cu" "B.Cu") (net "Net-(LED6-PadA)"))
 (segment (start 45.7949 36.1974) (end 46.6783 35.314) (width 0.2) (layer "B.Cu") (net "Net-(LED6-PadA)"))
 (segment (start 35.4969 35.4805) (end 36.2138 36.1974) (width 0.2) (layer "B.Cu") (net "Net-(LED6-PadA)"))
 (segment (start 36.2138 36.1974) (end 45.7949 36.1974) (width 0.2) (layer "B.Cu") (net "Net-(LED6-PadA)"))
 (segment (start 37.4484 30) (end 39.7483 30) (width 0.2) (layer "F.Cu") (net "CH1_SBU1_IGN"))
 (segment (start 28.73 31.27) (end 29.9715 30.0285) (width 0.2) (layer "F.Cu") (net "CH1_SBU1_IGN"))
 (segment (start 35.65 33.15) (end 35.65 32.5483) (width 0.2) (layer "F.Cu") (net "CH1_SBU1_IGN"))
 (segment (start 37.05 31.3001) (end 37.05 30.3984) (width 0.2) (layer "F.Cu") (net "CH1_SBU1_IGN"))
 (segment (start 37.05 30.3984) (end 37.4484 30) (width 0.2) (layer "F.Cu") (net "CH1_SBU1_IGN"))
 (segment (start 37.05 31.3001) (end 37.05 32.2018) (width 0.2) (layer "F.Cu") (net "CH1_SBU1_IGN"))
 (segment (start 35.6956 30.0285) (end 36.0655 30.3984) (width 0.2) (layer "F.Cu") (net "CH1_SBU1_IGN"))
 (segment (start 29.9715 30.0285) (end 35.6956 30.0285) (width 0.2) (layer "F.Cu") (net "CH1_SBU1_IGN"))
 (segment (start 36.7035 32.5483) (end 37.05 32.2018) (width 0.2) (layer "F.Cu") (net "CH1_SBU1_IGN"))
 (segment (start 36.0655 30.3984) (end 37.05 30.3984) (width 0.2) (layer "F.Cu") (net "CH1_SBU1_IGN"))
 (segment (start 35.65 32.5483) (end 36.7035 32.5483) (width 0.2) (layer "F.Cu") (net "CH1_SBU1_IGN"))
 (segment (start 40.35 30) (end 39.7483 30) (width 0.2) (layer "F.Cu") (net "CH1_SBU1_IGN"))
 (segment (start 42 35.15) (end 40.3184 35.15) (width 0.2) (layer "F.Cu") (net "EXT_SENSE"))
 (segment (start 42.5483 36.3) (end 42.5483 35.6983) (width 0.2) (layer "F.Cu") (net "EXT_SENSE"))
 (segment (start 42.5483 35.6983) (end 42 35.15) (width 0.2) (layer "F.Cu") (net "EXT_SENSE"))
 (segment (start 43.15 36.3) (end 42.5483 36.3) (width 0.2) (layer "F.Cu") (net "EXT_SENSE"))
 (via (at 40.3184 35.15) (size 0.6) (drill 0.3) (layers "F.Cu" "B.Cu") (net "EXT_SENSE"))
 (segment (start 34.8433 27.4745) (end 36.7749 29.4061) (width 0.2) (layer "B.Cu") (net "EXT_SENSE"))
 (segment (start 32.5255 27.4745) (end 34.8433 27.4745) (width 0.2) (layer "B.Cu") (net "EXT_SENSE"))
 (segment (start 36.7749 29.4061) (end 36.7749 31.6065) (width 0.2) (layer "B.Cu") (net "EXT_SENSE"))
 (segment (start 36.7749 31.6065) (end 40.3184 35.15) (width 0.2) (layer "B.Cu") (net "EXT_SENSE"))
 (segment (start 31.27 28.73) (end 32.5255 27.4745) (width 0.2) (layer "B.Cu") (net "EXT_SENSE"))
 (segment (start 35.1483 34.15) (end 41.9483 34.15) (width 0.2) (layer "F.Cu") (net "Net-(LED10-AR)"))
 (segment (start 34.75 33.15) (end 34.75 33.7517) (width 0.2) (layer "F.Cu") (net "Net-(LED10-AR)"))
 (segment (start 42.65 34.15) (end 41.9483 34.15) (width 0.2) (layer "F.Cu") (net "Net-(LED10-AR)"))
 (segment (start 34.75 33.7517) (end 35.1483 34.15) (width 0.2) (layer "F.Cu") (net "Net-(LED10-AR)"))
 (segment (start 45.2517 34.15) (end 45.2517 33.7114) (width 0.2) (layer "F.Cu") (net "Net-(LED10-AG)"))
 (segment (start 45.2517 33.7114) (end 45.8174 33.1457) (width 0.2) (layer "F.Cu") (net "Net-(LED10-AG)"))
 (segment (start 45.8174 33.1457) (end 47.2865 33.1457) (width 0.2) (layer "F.Cu") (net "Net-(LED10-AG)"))
 (segment (start 45.9954 29.3983) (end 46.22 29.1737) (width 0.2) (layer "F.Cu") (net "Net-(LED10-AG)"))
 (segment (start 45.95 29.3983) (end 45.9954 29.3983) (width 0.2) (layer "F.Cu") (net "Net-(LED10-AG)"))
 (segment (start 44.55 34.15) (end 45.2517 34.15) (width 0.2) (layer "F.Cu") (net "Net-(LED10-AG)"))
 (segment (start 45.95 30) (end 45.95 29.3983) (width 0.2) (layer "F.Cu") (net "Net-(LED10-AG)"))
 (via (at 46.22 29.1737) (size 0.6) (drill 0.3) (layers "F.Cu" "B.Cu") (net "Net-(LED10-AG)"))
 (via (at 47.2865 33.1457) (size 0.6) (drill 0.3) (layers "F.Cu" "B.Cu") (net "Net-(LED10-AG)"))
 (segment (start 46.22 32.0792) (end 47.2865 33.1457) (width 0.2) (layer "B.Cu") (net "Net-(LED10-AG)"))
 (segment (start 46.22 29.1737) (end 46.22 32.0792) (width 0.2) (layer "B.Cu") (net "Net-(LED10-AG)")))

